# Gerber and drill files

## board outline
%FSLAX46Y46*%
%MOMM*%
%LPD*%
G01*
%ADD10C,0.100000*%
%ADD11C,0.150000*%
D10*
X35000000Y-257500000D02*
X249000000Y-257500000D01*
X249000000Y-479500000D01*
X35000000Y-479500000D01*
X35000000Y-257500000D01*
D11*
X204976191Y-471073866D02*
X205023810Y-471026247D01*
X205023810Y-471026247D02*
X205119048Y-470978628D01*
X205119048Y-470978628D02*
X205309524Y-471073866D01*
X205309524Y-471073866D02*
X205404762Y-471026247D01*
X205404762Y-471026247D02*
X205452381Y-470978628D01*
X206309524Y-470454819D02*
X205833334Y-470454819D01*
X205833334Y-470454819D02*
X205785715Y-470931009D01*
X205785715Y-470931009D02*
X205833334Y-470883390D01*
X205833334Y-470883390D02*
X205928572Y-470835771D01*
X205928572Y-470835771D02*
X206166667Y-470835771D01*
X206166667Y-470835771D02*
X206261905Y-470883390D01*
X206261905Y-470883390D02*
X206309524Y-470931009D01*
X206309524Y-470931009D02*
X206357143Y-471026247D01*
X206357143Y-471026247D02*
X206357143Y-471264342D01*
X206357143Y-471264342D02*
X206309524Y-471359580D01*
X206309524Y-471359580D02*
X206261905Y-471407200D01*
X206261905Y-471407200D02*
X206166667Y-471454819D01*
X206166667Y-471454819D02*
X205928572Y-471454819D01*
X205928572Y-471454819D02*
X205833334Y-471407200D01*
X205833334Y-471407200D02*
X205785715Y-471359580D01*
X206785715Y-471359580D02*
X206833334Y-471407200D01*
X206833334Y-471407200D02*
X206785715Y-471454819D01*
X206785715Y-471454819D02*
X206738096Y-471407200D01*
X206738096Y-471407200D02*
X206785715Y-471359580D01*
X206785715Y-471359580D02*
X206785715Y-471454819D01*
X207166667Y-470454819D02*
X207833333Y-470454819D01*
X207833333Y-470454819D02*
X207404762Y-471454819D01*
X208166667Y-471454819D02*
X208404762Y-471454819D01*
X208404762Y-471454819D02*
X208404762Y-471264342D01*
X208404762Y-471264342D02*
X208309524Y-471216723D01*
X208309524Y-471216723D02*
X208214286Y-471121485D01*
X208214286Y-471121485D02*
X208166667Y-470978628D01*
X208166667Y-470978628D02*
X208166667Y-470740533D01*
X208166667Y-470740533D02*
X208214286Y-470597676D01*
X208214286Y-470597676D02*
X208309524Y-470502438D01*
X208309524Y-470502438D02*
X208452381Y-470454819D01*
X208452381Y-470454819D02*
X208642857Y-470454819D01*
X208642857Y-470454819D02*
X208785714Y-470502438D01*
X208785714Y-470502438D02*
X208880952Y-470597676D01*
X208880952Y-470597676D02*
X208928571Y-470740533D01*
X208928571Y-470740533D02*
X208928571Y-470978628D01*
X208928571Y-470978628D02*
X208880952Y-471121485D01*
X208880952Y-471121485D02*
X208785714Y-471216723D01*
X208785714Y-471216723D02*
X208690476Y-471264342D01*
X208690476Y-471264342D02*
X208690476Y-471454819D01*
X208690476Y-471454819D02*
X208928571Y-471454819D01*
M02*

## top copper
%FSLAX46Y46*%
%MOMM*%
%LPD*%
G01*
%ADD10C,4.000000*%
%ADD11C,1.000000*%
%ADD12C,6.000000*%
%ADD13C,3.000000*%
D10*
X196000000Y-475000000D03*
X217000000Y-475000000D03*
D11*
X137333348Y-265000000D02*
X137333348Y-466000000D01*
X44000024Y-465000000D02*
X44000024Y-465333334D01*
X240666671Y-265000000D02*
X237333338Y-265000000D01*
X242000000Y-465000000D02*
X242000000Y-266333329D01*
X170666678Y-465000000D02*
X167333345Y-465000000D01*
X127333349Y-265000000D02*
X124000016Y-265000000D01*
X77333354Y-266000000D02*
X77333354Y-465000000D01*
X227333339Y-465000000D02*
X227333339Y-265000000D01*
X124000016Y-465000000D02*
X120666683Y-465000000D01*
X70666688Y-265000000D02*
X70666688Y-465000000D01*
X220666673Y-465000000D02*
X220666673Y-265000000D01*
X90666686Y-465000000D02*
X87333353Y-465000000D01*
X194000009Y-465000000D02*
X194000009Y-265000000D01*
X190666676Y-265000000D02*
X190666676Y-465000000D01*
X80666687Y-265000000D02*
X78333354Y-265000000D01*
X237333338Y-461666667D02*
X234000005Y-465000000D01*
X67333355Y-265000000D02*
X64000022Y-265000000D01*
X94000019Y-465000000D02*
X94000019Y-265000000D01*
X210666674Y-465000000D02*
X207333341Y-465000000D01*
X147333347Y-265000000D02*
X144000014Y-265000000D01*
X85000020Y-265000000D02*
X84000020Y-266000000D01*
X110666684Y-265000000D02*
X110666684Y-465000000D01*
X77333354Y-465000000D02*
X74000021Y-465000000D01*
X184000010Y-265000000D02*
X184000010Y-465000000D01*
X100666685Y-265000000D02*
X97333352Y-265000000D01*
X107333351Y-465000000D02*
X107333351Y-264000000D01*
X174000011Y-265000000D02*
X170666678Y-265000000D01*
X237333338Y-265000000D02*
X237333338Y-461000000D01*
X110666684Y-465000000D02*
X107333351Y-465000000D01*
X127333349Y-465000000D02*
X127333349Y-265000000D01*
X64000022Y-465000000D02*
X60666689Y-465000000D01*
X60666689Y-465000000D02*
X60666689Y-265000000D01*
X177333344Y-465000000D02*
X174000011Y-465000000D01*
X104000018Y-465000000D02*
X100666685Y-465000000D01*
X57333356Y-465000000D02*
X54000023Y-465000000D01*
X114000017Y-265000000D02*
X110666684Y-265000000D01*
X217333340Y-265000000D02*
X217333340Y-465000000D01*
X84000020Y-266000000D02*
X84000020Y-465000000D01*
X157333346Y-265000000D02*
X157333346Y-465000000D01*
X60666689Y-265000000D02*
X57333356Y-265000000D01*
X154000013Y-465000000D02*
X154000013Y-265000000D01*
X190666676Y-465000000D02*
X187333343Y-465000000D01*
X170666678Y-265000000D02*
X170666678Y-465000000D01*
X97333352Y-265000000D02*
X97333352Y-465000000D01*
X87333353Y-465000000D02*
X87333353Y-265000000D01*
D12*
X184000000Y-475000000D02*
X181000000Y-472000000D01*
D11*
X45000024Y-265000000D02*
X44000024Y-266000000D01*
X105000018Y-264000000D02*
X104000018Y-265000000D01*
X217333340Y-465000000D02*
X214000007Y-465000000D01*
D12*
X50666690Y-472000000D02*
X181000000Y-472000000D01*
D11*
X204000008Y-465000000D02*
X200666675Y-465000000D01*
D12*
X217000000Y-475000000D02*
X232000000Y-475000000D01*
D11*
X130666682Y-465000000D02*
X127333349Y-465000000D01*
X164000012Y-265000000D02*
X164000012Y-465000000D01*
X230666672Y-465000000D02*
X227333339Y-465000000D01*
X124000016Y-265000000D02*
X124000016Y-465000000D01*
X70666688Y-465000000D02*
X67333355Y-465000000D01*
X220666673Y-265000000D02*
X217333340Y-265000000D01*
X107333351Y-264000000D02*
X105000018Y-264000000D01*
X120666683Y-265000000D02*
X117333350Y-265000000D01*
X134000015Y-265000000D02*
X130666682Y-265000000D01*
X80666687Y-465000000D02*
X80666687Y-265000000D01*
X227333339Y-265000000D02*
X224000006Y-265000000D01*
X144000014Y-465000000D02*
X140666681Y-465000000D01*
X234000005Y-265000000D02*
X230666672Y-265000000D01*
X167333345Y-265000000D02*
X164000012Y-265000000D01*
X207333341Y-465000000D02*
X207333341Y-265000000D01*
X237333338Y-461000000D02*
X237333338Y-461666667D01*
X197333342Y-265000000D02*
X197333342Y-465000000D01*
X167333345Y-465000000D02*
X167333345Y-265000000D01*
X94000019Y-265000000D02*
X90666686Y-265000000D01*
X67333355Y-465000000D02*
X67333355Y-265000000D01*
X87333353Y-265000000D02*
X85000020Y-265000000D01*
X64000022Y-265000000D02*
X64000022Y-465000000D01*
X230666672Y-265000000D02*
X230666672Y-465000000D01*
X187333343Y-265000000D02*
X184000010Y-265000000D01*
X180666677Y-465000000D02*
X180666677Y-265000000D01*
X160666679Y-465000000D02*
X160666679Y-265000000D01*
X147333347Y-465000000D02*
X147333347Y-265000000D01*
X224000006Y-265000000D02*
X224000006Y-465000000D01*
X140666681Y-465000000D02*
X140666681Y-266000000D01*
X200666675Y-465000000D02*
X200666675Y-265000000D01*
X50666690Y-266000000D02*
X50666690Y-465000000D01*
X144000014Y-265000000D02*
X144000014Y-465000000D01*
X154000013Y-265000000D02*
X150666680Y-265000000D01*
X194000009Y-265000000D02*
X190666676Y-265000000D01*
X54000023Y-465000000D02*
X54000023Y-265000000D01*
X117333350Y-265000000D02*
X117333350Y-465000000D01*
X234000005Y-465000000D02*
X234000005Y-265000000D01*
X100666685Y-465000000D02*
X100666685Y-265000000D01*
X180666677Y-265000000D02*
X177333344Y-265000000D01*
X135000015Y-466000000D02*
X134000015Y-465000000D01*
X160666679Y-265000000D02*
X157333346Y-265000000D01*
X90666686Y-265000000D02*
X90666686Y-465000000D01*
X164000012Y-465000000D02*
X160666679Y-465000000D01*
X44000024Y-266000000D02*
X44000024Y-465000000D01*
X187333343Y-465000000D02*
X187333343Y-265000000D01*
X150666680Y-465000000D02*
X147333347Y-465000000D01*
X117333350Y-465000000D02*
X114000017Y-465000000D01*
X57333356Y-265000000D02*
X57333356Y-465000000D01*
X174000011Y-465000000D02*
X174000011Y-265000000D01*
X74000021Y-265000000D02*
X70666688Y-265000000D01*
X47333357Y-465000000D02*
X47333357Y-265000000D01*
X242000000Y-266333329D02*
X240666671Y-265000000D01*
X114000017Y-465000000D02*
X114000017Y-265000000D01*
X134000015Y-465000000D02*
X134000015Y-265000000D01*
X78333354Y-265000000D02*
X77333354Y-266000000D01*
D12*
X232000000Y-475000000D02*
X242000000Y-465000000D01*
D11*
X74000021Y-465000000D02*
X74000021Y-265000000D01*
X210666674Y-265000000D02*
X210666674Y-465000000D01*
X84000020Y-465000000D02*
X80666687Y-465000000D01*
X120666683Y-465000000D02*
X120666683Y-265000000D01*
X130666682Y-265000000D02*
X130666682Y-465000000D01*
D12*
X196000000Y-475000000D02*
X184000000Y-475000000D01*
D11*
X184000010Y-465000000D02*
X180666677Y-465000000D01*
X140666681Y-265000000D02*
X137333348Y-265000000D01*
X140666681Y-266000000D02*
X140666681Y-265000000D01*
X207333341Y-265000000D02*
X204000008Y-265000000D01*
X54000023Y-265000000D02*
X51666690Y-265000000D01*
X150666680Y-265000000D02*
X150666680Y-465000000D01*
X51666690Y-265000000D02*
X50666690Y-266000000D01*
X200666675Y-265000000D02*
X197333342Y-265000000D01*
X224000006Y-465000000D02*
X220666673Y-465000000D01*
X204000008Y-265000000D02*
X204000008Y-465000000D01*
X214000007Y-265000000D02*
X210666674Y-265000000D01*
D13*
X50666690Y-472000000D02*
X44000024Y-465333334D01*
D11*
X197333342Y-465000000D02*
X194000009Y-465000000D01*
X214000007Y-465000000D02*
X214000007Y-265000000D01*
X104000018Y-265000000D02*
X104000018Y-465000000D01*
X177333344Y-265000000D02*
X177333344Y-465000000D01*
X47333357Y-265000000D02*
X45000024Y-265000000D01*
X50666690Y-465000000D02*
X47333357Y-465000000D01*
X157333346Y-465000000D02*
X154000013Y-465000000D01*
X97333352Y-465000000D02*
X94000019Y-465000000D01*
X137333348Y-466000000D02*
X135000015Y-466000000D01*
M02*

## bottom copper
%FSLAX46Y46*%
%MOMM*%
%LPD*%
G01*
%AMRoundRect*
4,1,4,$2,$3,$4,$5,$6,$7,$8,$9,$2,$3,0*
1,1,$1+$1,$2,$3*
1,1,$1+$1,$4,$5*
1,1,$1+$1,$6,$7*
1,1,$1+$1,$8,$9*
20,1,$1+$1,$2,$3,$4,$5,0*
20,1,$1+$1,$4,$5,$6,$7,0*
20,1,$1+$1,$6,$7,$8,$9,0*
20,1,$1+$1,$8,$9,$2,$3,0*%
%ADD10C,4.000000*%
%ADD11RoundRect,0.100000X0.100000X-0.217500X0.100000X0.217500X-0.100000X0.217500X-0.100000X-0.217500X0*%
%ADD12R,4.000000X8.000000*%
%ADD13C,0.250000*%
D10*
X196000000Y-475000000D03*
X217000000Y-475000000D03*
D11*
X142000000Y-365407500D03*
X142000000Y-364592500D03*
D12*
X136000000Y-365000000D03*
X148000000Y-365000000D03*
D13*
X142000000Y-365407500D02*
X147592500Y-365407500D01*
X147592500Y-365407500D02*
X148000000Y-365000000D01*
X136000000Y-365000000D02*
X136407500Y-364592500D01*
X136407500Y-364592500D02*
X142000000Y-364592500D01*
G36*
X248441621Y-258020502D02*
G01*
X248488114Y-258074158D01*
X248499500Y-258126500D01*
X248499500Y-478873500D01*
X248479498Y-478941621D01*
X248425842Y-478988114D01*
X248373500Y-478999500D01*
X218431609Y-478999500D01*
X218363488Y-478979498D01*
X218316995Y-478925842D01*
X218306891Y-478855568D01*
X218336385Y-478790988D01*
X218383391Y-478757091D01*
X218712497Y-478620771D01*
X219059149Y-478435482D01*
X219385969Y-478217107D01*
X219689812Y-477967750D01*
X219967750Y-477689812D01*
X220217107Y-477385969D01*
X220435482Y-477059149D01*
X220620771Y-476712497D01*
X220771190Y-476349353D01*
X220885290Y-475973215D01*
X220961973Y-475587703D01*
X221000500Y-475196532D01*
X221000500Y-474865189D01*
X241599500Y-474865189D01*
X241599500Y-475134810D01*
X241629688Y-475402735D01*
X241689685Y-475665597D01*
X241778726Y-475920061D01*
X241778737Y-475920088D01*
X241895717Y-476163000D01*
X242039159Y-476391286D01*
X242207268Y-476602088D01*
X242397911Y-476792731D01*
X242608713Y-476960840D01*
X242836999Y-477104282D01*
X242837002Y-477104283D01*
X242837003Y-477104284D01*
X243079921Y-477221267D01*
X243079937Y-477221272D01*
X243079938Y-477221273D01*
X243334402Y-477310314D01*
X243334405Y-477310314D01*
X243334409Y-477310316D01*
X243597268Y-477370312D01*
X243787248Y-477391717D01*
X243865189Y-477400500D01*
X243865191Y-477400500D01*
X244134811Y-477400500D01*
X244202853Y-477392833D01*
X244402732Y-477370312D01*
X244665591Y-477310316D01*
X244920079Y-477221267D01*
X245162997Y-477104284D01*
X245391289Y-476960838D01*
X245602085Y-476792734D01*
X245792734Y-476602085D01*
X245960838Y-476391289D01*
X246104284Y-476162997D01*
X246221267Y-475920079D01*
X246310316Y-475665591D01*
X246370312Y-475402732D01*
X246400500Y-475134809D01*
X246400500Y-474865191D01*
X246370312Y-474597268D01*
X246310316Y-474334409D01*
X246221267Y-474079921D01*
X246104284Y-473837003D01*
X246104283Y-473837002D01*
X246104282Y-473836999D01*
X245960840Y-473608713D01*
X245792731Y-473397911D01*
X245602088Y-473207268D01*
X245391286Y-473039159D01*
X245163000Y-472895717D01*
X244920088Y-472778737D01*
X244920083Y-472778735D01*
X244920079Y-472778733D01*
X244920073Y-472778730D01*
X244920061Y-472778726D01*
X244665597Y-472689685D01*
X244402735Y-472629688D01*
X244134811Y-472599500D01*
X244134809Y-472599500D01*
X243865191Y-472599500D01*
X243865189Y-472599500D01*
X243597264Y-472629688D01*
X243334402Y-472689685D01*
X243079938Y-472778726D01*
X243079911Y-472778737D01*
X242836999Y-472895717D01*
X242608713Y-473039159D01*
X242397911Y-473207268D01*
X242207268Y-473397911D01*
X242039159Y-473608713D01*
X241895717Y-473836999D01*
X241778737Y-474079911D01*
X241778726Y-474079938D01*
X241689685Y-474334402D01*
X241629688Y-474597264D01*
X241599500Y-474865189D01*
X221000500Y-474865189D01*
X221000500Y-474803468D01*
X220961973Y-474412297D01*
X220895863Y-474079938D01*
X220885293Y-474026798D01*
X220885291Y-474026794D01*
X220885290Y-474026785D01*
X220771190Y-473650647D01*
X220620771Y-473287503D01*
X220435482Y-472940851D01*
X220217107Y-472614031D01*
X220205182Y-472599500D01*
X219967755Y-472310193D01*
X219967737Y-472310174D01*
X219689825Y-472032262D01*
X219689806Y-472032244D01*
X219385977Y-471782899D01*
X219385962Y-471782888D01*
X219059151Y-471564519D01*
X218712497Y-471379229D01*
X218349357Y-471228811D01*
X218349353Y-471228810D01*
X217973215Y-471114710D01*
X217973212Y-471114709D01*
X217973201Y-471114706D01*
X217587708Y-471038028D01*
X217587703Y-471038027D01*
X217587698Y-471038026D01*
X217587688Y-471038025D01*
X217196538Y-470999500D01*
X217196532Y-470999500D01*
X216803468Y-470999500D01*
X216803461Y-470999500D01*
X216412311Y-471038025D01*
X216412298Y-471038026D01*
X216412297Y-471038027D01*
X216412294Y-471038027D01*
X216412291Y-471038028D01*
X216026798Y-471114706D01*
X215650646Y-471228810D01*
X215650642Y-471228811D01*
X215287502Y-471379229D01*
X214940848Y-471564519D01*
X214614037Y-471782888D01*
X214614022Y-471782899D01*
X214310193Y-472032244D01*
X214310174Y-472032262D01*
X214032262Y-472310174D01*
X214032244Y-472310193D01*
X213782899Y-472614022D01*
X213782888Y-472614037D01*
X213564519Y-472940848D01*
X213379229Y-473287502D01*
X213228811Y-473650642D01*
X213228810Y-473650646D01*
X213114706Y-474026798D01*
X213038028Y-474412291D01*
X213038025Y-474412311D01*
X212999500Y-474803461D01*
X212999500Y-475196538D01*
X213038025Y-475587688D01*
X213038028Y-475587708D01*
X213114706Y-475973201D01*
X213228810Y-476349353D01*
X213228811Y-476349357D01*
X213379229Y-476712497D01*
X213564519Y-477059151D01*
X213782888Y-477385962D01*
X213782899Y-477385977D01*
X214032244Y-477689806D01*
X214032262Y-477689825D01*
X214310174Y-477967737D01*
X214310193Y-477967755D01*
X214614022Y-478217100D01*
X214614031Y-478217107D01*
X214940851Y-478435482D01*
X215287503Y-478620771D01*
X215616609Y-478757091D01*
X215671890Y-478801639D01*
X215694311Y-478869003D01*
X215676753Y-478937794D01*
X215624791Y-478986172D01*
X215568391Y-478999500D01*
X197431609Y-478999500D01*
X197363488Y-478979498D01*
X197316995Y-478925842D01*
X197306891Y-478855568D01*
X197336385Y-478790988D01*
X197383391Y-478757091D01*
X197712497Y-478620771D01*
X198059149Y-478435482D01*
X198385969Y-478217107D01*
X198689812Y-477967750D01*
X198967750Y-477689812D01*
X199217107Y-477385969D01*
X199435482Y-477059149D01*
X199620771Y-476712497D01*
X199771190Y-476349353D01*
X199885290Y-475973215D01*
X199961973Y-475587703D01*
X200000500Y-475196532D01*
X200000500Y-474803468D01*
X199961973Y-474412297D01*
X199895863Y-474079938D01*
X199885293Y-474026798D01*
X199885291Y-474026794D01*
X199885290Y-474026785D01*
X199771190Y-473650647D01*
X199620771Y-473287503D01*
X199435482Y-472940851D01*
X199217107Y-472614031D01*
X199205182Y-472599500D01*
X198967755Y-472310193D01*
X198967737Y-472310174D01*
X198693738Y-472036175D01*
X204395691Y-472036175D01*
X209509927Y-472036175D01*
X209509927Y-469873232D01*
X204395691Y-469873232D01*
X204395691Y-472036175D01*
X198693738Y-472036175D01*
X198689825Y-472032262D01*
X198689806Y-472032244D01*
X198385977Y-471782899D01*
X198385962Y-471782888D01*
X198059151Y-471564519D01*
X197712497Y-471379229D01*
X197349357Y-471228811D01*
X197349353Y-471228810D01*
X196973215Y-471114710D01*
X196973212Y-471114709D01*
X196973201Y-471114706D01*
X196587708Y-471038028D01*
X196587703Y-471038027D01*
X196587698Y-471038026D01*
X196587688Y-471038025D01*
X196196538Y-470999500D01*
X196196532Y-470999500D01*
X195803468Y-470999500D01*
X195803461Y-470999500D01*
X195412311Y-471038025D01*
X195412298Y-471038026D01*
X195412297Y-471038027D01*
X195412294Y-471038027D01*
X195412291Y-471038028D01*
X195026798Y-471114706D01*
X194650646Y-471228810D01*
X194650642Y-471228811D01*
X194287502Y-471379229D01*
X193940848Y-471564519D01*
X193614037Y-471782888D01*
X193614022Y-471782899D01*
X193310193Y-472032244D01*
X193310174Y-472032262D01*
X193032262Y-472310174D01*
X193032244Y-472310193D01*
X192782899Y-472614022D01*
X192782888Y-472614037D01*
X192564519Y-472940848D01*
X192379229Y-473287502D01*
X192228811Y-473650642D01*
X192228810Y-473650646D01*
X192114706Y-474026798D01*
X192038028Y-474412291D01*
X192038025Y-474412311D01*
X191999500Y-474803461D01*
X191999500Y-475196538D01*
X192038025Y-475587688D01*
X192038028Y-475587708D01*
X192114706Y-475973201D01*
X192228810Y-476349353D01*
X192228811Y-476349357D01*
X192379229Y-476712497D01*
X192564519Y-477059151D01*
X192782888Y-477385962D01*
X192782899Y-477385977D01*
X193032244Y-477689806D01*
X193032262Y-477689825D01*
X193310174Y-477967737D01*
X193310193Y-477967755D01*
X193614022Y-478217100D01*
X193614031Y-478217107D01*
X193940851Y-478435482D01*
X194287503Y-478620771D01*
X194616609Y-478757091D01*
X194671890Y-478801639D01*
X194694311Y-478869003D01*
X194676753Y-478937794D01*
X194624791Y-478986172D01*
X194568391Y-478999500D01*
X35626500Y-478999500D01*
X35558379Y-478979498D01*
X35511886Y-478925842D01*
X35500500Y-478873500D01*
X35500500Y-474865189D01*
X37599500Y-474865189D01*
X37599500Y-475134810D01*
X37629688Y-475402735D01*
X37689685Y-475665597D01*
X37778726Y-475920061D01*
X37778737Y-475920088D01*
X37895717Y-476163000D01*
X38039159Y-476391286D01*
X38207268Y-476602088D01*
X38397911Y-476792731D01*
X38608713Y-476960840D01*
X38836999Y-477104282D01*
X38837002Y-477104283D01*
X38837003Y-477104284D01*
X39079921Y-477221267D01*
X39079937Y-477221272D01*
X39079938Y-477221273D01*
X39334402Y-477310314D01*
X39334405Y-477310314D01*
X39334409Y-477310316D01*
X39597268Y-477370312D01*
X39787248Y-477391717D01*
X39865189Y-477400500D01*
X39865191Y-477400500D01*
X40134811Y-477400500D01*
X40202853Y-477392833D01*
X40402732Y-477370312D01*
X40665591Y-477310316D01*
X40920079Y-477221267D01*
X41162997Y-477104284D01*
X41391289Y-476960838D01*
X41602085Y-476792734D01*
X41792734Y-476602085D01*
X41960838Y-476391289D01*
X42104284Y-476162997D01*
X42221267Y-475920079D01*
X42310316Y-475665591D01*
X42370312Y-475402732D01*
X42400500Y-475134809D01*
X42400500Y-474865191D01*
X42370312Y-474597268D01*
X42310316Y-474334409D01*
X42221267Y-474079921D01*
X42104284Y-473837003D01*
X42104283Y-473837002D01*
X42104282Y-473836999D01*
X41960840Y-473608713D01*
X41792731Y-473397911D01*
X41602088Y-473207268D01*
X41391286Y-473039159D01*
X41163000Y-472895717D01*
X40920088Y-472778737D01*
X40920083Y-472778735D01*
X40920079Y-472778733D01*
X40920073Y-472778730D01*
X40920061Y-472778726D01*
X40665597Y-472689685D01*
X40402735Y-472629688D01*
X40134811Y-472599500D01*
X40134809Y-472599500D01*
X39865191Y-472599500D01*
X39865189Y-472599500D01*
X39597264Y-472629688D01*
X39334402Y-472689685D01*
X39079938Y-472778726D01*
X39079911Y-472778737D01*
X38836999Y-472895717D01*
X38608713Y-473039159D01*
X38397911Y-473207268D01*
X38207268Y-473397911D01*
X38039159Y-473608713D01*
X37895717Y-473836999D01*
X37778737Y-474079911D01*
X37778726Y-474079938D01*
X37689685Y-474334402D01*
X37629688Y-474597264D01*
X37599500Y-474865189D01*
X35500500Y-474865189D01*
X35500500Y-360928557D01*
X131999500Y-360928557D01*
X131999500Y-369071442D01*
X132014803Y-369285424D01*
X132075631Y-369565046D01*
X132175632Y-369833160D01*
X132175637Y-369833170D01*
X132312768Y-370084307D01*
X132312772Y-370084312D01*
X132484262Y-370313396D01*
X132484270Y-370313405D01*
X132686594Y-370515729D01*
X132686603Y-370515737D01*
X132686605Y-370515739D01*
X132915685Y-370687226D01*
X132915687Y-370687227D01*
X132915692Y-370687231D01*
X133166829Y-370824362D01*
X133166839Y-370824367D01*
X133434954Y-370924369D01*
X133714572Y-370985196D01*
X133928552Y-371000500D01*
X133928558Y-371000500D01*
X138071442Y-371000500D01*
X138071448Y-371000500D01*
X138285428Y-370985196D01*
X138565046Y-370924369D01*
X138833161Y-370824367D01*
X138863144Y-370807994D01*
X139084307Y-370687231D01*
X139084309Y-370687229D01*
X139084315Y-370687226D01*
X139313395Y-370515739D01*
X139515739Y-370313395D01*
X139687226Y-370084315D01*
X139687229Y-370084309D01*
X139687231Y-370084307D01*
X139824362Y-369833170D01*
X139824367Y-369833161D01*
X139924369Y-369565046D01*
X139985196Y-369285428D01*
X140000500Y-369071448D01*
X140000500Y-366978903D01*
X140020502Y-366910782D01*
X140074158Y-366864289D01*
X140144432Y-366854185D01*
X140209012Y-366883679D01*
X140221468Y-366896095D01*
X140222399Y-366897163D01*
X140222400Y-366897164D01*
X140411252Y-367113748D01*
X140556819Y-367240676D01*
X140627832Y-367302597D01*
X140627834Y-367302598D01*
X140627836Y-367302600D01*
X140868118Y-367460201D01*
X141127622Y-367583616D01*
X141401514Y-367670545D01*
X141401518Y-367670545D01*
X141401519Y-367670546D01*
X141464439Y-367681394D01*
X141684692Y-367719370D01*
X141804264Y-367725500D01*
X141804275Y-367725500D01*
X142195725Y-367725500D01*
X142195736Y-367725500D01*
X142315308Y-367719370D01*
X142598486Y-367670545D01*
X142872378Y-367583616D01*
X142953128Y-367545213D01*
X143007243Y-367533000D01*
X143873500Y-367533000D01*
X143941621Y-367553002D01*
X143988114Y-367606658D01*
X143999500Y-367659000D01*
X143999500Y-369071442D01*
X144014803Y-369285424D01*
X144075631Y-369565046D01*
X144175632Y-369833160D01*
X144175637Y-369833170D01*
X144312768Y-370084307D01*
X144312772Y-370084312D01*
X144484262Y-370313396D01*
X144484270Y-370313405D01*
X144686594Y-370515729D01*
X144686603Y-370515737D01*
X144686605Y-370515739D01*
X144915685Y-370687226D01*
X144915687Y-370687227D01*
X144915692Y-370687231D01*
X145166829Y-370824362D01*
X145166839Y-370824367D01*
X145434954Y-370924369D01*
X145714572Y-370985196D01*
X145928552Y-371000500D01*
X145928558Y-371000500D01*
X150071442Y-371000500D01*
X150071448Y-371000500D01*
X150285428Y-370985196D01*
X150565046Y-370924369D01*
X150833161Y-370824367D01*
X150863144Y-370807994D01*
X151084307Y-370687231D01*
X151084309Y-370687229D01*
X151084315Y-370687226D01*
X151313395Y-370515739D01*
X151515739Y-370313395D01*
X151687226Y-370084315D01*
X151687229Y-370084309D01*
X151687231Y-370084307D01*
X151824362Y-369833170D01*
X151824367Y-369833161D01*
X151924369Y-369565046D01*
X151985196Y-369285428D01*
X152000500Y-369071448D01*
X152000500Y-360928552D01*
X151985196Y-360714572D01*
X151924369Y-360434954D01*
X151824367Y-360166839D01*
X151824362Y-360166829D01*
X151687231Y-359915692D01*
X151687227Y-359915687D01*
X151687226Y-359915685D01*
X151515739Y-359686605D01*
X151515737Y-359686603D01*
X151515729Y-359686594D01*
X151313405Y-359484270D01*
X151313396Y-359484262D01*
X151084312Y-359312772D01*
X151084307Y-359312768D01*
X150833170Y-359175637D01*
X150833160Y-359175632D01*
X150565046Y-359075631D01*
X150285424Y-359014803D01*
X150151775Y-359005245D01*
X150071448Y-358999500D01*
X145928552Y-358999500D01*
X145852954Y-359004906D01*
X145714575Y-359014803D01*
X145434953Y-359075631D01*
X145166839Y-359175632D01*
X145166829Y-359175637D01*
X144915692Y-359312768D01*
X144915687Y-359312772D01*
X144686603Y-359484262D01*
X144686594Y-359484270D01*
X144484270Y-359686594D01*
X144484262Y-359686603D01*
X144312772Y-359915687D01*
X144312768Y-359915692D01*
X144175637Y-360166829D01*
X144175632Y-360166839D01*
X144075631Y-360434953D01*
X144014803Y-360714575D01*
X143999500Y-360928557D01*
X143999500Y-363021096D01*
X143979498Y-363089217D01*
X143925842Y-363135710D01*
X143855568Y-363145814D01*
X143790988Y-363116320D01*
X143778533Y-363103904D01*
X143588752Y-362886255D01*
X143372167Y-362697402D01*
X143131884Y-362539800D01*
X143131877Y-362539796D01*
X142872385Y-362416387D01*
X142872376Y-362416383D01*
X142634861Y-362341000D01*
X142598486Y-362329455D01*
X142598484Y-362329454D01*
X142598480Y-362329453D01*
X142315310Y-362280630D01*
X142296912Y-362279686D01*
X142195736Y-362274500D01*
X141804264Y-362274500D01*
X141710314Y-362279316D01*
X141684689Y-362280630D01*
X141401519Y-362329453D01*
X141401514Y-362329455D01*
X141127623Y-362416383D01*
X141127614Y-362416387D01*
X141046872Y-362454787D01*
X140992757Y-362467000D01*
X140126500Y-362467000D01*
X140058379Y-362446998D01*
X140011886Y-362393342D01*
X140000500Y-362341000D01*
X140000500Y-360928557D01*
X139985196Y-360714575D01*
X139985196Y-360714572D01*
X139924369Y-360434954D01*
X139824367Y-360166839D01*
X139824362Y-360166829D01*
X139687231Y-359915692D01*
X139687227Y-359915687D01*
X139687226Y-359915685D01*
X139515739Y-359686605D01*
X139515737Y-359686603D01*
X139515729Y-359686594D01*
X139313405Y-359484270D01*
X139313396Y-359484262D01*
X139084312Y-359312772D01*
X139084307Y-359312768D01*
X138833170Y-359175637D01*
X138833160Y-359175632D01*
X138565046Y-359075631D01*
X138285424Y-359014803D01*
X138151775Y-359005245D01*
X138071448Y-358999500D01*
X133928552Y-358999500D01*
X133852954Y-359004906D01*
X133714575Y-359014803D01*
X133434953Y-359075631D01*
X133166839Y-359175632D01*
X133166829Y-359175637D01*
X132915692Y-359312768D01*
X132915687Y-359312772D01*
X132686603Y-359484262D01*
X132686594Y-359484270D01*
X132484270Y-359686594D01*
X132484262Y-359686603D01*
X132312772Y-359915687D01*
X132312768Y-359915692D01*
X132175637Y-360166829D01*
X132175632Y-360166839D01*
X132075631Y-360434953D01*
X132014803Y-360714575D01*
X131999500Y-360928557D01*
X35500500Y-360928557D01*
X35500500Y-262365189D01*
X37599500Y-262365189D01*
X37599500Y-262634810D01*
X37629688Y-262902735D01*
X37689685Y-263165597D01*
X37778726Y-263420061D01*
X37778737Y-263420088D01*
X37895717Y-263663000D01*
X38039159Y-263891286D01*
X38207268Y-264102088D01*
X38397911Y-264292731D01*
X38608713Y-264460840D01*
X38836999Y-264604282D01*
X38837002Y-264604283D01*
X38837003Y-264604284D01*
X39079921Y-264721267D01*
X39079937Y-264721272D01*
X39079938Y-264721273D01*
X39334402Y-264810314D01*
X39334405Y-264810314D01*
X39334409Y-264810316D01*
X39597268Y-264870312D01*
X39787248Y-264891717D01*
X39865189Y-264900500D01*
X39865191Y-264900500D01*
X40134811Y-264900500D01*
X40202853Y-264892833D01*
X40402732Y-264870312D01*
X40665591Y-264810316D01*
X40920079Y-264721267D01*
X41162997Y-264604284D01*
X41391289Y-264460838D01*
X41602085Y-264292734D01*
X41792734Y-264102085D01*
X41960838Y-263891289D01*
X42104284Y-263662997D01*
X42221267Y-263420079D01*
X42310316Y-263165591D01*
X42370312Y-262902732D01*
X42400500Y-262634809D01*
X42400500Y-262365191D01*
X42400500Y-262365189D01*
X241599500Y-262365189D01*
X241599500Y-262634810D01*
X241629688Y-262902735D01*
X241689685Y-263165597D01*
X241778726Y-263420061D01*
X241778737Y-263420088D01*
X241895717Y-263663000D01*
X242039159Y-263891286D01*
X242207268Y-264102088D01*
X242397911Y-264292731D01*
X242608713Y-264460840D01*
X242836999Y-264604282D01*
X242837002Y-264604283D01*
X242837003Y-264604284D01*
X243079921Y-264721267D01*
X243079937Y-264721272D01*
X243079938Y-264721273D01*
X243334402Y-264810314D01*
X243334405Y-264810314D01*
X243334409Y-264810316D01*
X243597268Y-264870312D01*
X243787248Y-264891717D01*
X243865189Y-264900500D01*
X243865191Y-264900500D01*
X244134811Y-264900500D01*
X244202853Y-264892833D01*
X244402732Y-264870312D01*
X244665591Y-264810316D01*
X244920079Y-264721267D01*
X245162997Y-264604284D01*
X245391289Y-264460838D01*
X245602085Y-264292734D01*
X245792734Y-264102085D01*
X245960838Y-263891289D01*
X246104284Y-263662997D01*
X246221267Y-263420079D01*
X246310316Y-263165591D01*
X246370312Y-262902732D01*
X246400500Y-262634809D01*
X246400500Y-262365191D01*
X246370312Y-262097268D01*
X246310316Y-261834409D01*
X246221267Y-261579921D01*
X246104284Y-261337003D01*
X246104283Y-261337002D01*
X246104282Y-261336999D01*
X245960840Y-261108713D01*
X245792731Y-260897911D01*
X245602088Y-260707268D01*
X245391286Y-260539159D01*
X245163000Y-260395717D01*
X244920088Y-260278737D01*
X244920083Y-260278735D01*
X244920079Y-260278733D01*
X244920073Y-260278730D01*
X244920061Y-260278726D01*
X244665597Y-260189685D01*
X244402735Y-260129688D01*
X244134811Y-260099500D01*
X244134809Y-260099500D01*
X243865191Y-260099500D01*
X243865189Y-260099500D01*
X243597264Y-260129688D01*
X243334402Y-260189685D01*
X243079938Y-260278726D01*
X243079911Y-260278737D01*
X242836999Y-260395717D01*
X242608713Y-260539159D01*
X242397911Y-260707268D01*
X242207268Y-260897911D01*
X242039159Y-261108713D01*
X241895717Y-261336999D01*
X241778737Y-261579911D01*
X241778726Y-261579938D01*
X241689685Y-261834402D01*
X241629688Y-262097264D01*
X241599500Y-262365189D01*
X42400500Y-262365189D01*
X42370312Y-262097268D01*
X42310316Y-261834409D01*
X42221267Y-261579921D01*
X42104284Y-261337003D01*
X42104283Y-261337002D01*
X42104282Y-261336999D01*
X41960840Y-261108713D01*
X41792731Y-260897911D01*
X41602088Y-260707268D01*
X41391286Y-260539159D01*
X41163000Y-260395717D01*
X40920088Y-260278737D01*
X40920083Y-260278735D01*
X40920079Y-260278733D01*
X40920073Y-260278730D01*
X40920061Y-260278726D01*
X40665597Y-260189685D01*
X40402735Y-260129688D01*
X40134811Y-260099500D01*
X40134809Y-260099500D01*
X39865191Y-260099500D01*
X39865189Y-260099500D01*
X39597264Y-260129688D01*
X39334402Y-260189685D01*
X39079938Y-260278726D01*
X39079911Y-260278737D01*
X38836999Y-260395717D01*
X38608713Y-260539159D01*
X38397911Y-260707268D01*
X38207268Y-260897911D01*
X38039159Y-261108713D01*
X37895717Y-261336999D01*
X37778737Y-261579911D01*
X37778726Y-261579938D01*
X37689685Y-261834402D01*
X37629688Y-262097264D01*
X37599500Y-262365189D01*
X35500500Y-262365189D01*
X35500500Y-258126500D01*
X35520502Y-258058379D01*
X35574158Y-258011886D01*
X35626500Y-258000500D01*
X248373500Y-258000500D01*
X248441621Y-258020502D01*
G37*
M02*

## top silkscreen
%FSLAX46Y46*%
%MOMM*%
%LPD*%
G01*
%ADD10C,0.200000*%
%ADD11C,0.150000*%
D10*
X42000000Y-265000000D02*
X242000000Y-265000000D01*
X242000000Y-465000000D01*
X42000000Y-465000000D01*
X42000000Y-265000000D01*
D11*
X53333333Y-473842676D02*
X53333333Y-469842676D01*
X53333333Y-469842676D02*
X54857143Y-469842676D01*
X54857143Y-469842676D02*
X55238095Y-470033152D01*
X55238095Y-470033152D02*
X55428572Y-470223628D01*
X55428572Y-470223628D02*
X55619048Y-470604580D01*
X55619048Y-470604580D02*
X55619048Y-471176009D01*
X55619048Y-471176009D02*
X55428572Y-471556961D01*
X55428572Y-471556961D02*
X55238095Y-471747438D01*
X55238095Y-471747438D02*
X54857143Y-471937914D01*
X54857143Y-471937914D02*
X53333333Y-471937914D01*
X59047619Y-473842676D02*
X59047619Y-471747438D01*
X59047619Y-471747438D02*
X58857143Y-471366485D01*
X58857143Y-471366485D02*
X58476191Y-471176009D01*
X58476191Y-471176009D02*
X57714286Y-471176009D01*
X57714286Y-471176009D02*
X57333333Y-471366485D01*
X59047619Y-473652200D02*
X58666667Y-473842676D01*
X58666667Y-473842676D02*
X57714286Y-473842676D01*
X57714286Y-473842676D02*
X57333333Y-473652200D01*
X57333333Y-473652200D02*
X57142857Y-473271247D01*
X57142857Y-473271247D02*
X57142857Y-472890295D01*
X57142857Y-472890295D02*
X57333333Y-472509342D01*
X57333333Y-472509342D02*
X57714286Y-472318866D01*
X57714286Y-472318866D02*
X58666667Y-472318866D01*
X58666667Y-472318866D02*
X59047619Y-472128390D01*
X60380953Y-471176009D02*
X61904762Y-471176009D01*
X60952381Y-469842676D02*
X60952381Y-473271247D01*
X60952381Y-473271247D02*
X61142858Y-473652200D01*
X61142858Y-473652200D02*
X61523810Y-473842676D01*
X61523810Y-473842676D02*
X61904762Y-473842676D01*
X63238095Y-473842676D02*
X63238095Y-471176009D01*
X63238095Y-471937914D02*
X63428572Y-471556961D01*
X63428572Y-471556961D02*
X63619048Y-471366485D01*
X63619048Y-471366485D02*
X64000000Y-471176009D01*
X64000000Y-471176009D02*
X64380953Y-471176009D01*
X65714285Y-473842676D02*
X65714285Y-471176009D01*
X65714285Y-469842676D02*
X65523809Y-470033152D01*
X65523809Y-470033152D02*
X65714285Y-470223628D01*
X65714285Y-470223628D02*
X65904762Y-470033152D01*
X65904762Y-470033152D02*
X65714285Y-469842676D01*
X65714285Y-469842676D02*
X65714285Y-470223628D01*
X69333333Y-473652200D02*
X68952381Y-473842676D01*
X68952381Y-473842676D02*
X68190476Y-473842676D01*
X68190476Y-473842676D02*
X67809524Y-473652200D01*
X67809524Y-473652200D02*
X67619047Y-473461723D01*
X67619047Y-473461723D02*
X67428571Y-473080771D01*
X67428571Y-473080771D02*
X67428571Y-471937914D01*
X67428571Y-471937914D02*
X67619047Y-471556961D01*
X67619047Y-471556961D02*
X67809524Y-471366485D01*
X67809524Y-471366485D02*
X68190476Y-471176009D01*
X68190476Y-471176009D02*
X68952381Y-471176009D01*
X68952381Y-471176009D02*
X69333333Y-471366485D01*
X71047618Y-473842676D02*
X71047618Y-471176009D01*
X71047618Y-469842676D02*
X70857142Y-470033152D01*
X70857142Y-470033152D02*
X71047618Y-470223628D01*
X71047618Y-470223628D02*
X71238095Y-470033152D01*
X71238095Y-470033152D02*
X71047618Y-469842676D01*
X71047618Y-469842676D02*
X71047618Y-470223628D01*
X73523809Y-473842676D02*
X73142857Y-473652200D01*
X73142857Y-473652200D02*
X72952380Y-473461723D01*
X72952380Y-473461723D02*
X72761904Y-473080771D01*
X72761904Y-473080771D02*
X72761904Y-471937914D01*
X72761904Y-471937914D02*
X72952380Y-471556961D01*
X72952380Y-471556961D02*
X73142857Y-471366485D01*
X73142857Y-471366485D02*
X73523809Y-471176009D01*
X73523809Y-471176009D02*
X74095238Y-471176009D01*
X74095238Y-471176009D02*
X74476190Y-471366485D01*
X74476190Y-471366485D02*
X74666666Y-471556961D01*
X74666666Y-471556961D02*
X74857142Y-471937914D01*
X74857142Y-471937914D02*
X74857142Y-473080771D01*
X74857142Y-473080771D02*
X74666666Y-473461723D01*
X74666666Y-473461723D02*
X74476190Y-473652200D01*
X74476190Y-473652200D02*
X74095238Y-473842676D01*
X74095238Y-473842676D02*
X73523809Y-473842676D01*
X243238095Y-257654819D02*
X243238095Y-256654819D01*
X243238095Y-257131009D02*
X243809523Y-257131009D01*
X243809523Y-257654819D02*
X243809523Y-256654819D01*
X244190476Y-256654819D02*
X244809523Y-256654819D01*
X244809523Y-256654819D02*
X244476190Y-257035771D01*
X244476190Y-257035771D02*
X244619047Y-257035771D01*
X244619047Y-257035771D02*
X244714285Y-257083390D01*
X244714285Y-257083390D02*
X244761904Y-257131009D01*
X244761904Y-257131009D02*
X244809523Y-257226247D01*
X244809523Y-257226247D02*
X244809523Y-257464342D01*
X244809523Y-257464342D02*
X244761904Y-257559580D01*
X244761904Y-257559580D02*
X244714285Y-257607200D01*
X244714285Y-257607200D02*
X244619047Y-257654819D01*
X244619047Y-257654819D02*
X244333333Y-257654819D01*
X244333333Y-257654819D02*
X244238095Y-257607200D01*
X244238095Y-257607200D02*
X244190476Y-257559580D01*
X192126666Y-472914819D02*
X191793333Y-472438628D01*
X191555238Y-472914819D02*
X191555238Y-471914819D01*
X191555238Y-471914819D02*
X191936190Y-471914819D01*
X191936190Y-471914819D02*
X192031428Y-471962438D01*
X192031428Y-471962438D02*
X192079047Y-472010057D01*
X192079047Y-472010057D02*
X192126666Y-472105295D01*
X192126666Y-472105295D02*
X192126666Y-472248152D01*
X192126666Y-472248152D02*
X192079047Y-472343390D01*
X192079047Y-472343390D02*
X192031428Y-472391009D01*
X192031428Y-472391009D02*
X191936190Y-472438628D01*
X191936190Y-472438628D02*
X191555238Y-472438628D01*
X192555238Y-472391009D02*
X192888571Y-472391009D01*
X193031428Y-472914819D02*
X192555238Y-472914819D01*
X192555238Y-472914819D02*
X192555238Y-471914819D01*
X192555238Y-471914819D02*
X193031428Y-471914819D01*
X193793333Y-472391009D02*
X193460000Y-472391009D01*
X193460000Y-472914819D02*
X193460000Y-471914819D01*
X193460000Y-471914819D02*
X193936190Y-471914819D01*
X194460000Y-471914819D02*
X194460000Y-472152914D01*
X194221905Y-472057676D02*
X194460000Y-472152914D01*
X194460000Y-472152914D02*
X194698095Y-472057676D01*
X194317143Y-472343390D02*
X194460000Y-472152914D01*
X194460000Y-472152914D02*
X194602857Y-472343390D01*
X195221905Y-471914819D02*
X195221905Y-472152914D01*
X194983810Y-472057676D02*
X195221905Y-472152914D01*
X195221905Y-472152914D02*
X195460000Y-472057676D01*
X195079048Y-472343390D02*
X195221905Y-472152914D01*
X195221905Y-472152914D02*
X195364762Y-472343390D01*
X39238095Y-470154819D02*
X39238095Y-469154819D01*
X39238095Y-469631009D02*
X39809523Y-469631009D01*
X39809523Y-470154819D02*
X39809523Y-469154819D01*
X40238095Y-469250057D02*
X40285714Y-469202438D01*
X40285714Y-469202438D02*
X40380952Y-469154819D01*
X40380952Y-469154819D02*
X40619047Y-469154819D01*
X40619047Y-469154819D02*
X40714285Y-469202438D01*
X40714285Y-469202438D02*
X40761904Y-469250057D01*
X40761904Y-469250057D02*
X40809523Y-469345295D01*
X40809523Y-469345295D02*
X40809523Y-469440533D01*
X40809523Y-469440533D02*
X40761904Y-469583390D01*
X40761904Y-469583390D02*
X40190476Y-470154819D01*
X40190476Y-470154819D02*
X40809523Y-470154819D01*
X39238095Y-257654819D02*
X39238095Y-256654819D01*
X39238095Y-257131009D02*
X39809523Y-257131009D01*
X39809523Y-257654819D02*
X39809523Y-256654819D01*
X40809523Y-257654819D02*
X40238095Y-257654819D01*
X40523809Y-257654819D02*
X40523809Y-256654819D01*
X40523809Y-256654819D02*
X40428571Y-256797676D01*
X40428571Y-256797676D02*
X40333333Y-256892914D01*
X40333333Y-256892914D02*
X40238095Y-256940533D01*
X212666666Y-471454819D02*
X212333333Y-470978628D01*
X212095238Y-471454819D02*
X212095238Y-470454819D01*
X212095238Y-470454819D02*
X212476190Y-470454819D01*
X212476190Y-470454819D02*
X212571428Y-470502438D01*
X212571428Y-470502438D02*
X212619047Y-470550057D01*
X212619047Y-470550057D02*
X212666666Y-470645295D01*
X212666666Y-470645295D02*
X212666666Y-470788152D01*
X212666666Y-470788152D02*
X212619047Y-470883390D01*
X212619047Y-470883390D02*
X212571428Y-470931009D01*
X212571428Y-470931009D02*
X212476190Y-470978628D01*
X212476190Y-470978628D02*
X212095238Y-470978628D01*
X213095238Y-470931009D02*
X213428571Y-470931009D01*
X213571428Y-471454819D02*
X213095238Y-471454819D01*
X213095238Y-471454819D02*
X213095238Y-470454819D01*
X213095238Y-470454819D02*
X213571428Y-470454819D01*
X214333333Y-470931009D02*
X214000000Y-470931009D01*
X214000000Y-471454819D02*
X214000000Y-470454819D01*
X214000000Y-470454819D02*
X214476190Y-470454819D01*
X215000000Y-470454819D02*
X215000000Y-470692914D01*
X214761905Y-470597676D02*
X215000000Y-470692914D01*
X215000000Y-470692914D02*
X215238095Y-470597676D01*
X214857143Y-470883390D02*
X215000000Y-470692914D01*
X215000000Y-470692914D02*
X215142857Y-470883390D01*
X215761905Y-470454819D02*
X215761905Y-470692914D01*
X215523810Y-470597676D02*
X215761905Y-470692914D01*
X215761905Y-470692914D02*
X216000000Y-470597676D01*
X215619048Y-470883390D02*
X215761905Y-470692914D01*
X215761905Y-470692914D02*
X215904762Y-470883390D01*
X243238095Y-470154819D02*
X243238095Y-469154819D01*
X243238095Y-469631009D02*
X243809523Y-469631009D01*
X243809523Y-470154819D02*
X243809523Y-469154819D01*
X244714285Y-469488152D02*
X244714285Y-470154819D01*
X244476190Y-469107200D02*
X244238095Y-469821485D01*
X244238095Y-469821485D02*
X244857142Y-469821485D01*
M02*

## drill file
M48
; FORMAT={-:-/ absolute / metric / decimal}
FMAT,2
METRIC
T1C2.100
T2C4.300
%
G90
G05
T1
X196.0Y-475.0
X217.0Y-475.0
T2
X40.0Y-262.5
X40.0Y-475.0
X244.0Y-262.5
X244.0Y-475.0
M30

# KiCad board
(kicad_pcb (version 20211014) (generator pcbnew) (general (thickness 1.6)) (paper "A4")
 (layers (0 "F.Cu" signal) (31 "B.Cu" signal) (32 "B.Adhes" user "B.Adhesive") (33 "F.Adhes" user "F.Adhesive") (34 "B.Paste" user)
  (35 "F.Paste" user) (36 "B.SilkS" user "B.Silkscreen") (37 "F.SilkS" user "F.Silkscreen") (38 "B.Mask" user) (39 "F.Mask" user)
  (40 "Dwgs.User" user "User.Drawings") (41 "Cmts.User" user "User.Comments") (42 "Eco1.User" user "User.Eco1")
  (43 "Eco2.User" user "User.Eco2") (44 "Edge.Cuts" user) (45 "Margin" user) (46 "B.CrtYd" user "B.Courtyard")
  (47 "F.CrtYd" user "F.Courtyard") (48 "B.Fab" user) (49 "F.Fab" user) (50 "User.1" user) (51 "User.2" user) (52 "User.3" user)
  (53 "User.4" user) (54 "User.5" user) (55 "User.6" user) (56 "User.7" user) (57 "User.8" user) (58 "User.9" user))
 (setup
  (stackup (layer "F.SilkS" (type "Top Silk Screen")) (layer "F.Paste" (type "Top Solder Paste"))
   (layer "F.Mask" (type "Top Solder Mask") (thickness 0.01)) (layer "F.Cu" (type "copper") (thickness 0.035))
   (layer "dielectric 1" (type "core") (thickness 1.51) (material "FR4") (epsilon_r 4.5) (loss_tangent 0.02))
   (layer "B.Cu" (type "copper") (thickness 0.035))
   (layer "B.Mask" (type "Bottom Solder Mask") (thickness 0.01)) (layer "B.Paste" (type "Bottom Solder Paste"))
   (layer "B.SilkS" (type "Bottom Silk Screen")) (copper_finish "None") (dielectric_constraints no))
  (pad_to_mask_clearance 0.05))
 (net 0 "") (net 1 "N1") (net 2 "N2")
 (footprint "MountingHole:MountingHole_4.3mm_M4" (layer "F.Cu") (at 244 262.5)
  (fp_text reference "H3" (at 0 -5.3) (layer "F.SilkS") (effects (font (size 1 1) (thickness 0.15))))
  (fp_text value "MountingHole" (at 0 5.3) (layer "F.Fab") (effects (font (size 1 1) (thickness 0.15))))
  (pad "" np_thru_hole circle (at 0 0) (size 4.3 4.3) (drill 4.3) (layers *.Cu *.Mask)))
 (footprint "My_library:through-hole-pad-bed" (layer "F.Cu") (at 196 475)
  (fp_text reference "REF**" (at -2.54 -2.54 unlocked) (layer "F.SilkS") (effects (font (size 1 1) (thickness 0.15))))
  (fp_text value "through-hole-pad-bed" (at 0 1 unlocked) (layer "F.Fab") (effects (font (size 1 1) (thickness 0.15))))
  (pad "1" thru_hole circle (at 0 0) (size 4 4) (drill 2.1) (layers *.Cu *.Mask)))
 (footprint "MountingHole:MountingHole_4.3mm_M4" (layer "F.Cu") (at 40 475)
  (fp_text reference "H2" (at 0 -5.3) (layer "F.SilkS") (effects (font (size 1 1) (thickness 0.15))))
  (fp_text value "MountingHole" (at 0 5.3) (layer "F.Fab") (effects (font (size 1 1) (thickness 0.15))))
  (pad "" np_thru_hole circle (at 0 0) (size 4.3 4.3) (drill 4.3) (layers *.Cu *.Mask)))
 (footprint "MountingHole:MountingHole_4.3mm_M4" (layer "F.Cu") (at 40 262.5)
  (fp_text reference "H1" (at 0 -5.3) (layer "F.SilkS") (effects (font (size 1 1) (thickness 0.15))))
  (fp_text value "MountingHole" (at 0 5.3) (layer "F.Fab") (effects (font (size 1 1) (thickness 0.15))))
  (pad "" np_thru_hole circle (at 0 0) (size 4.3 4.3) (drill 4.3) (layers *.Cu *.Mask)))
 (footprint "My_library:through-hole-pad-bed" (layer "F.Cu") (at 217 475)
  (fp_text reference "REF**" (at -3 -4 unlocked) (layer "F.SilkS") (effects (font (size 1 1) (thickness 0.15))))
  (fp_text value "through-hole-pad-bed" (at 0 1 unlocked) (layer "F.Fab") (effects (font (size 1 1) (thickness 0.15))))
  (pad "1" thru_hole circle (at 0 0) (size 4 4) (drill 2.1) (layers *.Cu *.Mask)))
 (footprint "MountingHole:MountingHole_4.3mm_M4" (layer "F.Cu") (at 244 475)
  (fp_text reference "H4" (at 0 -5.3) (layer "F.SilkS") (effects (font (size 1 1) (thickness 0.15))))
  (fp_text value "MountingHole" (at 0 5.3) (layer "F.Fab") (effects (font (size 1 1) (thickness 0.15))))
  (pad "" np_thru_hole circle (at 0 0) (size 4.3 4.3) (drill 4.3) (layers *.Cu *.Mask)))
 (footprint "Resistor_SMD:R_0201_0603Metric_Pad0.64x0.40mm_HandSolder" (layer "B.Cu") (at 142 365 90)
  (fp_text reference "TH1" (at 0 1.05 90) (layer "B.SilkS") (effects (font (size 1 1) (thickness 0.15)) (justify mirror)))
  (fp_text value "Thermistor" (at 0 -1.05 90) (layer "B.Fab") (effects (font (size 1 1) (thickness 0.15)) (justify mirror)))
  (pad "" smd roundrect (at 0.4325 0 90) (size 0.458 0.36) (layers "B.Paste") (roundrect_rratio 0.25))
  (pad "" smd roundrect (at -0.4325 0 90) (size 0.458 0.36) (layers "B.Paste") (roundrect_rratio 0.25))
  (pad "1" smd roundrect (at -0.4075 0 90) (size 0.635 0.4) (layers "B.Cu" "B.Mask") (roundrect_rratio 0.25) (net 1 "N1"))
  (pad "2" smd roundrect (at 0.4075 0 90) (size 0.635 0.4) (layers "B.Cu" "B.Mask") (roundrect_rratio 0.25) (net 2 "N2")))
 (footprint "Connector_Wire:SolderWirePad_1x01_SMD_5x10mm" (layer "B.Cu") (at 136 365 180)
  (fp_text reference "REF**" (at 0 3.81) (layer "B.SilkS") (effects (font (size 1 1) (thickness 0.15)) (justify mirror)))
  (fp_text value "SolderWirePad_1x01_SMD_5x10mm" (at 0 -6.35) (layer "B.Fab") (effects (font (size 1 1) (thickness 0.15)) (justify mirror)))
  (pad "1" smd rect (at 0 0 180) (size 4 8) (layers "B.Cu" "B.Paste" "B.Mask") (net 2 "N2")))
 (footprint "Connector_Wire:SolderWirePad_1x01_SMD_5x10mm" (layer "B.Cu") (at 148 365 180)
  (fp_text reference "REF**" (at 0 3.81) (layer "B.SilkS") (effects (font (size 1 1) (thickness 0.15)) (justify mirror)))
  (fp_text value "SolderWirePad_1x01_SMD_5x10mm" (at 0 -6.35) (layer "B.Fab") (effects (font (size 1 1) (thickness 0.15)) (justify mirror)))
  (pad "1" smd rect (at 0 0 180) (size 4 8) (layers "B.Cu" "B.Paste" "B.Mask") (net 1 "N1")))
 (gr_rect (start 42 465) (end 242 265) (layer "F.SilkS") (width 0.2) (fill none))
 (gr_rect (start 249 257.5) (end 35 479.5) (layer "Edge.Cuts") (width 0.1) (fill none))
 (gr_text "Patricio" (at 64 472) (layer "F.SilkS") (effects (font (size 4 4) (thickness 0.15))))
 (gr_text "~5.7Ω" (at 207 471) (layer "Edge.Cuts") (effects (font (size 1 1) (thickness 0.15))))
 (segment (start 137.333348 265) (end 137.333348 466) (width 1) (layer "F.Cu") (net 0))
 (segment (start 44.000024 465) (end 44.000024 465.333334) (width 1) (layer "F.Cu") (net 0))
 (segment (start 240.666671 265) (end 237.333338 265) (width 1) (layer "F.Cu") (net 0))
 (segment (start 242 465) (end 242 266.333329) (width 1) (layer "F.Cu") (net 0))
 (segment (start 170.666678 465) (end 167.333345 465) (width 1) (layer "F.Cu") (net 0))
 (segment (start 127.333349 265) (end 124.000016 265) (width 1) (layer "F.Cu") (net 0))
 (segment (start 77.333354 266) (end 77.333354 465) (width 1) (layer "F.Cu") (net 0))
 (segment (start 227.333339 465) (end 227.333339 265) (width 1) (layer "F.Cu") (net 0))
 (segment (start 124.000016 465) (end 120.666683 465) (width 1) (layer "F.Cu") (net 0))
 (segment (start 70.666688 265) (end 70.666688 465) (width 1) (layer "F.Cu") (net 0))
 (segment (start 220.666673 465) (end 220.666673 265) (width 1) (layer "F.Cu") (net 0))
 (segment (start 90.666686 465) (end 87.333353 465) (width 1) (layer "F.Cu") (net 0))
 (segment (start 194.000009 465) (end 194.000009 265) (width 1) (layer "F.Cu") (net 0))
 (segment (start 190.666676 265) (end 190.666676 465) (width 1) (layer "F.Cu") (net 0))
 (segment (start 80.666687 265) (end 78.333354 265) (width 1) (layer "F.Cu") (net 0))
 (segment (start 237.333338 461.666667) (end 234.000005 465) (width 1) (layer "F.Cu") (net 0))
 (segment (start 67.333355 265) (end 64.000022 265) (width 1) (layer "F.Cu") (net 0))
 (segment (start 94.000019 465) (end 94.000019 265) (width 1) (layer "F.Cu") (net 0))
 (segment (start 210.666674 465) (end 207.333341 465) (width 1) (layer "F.Cu") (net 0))
 (segment (start 147.333347 265) (end 144.000014 265) (width 1) (layer "F.Cu") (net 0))
 (segment (start 85.00002 265) (end 84.00002 266) (width 1) (layer "F.Cu") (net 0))
 (segment (start 110.666684 265) (end 110.666684 465) (width 1) (layer "F.Cu") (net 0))
 (segment (start 77.333354 465) (end 74.000021 465) (width 1) (layer "F.Cu") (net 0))
 (segment (start 184.00001 265) (end 184.00001 465) (width 1) (layer "F.Cu") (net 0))
 (segment (start 100.666685 265) (end 97.333352 265) (width 1) (layer "F.Cu") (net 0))
 (segment (start 107.333351 465) (end 107.333351 264) (width 1) (layer "F.Cu") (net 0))
 (segment (start 174.000011 265) (end 170.666678 265) (width 1) (layer "F.Cu") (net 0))
 (segment (start 237.333338 265) (end 237.333338 461) (width 1) (layer "F.Cu") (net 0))
 (segment (start 110.666684 465) (end 107.333351 465) (width 1) (layer "F.Cu") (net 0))
 (segment (start 127.333349 465) (end 127.333349 265) (width 1) (layer "F.Cu") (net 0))
 (segment (start 64.000022 465) (end 60.666689 465) (width 1) (layer "F.Cu") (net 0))
 (segment (start 60.666689 465) (end 60.666689 265) (width 1) (layer "F.Cu") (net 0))
 (segment (start 177.333344 465) (end 174.000011 465) (width 1) (layer "F.Cu") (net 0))
 (segment (start 104.000018 465) (end 100.666685 465) (width 1) (layer "F.Cu") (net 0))
 (segment (start 57.333356 465) (end 54.000023 465) (width 1) (layer "F.Cu") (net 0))
 (segment (start 114.000017 265) (end 110.666684 265) (width 1) (layer "F.Cu") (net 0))
 (segment (start 217.33334 265) (end 217.33334 465) (width 1) (layer "F.Cu") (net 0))
 (segment (start 84.00002 266) (end 84.00002 465) (width 1) (layer "F.Cu") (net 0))
 (segment (start 157.333346 265) (end 157.333346 465) (width 1) (layer "F.Cu") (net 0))
 (segment (start 60.666689 265) (end 57.333356 265) (width 1) (layer "F.Cu") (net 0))
 (segment (start 154.000013 465) (end 154.000013 265) (width 1) (layer "F.Cu") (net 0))
 (segment (start 190.666676 465) (end 187.333343 465) (width 1) (layer "F.Cu") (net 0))
 (segment (start 170.666678 265) (end 170.666678 465) (width 1) (layer "F.Cu") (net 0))
 (segment (start 97.333352 265) (end 97.333352 465) (width 1) (layer "F.Cu") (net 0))
 (segment (start 87.333353 465) (end 87.333353 265) (width 1) (layer "F.Cu") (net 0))
 (segment (start 184 475) (end 181 472) (width 6) (layer "F.Cu") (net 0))
 (segment (start 45.000024 265) (end 44.000024 266) (width 1) (layer "F.Cu") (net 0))
 (segment (start 105.000018 264) (end 104.000018 265) (width 1) (layer "F.Cu") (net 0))
 (segment (start 217.33334 465) (end 214.000007 465) (width 1) (layer "F.Cu") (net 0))
 (segment (start 50.66669 472) (end 181 472) (width 6) (layer "F.Cu") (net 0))
 (segment (start 204.000008 465) (end 200.666675 465) (width 1) (layer "F.Cu") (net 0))
 (segment (start 217 475) (end 232 475) (width 6) (layer "F.Cu") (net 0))
 (segment (start 130.666682 465) (end 127.333349 465) (width 1) (layer "F.Cu") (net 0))
 (segment (start 164.000012 265) (end 164.000012 465) (width 1) (layer "F.Cu") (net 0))
 (segment (start 230.666672 465) (end 227.333339 465) (width 1) (layer "F.Cu") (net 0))
 (segment (start 124.000016 265) (end 124.000016 465) (width 1) (layer "F.Cu") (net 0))
 (segment (start 70.666688 465) (end 67.333355 465) (width 1) (layer "F.Cu") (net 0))
 (segment (start 220.666673 265) (end 217.33334 265) (width 1) (layer "F.Cu") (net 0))
 (segment (start 107.333351 264) (end 105.000018 264) (width 1) (layer "F.Cu") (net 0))
 (segment (start 120.666683 265) (end 117.33335 265) (width 1) (layer "F.Cu") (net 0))
 (segment (start 134.000015 265) (end 130.666682 265) (width 1) (layer "F.Cu") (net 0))
 (segment (start 80.666687 465) (end 80.666687 265) (width 1) (layer "F.Cu") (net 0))
 (segment (start 227.333339 265) (end 224.000006 265) (width 1) (layer "F.Cu") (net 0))
 (segment (start 144.000014 465) (end 140.666681 465) (width 1) (layer "F.Cu") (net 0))
 (segment (start 234.000005 265) (end 230.666672 265) (width 1) (layer "F.Cu") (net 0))
 (segment (start 167.333345 265) (end 164.000012 265) (width 1) (layer "F.Cu") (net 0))
 (segment (start 207.333341 465) (end 207.333341 265) (width 1) (layer "F.Cu") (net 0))
 (segment (start 237.333338 461) (end 237.333338 461.666667) (width 1) (layer "F.Cu") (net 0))
 (segment (start 197.333342 265) (end 197.333342 465) (width 1) (layer "F.Cu") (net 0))
 (segment (start 167.333345 465) (end 167.333345 265) (width 1) (layer "F.Cu") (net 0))
 (segment (start 94.000019 265) (end 90.666686 265) (width 1) (layer "F.Cu") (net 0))
 (segment (start 67.333355 465) (end 67.333355 265) (width 1) (layer "F.Cu") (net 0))
 (segment (start 87.333353 265) (end 85.00002 265) (width 1) (layer "F.Cu") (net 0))
 (segment (start 64.000022 265) (end 64.000022 465) (width 1) (layer "F.Cu") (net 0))
 (segment (start 230.666672 265) (end 230.666672 465) (width 1) (layer "F.Cu") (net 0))
 (segment (start 187.333343 265) (end 184.00001 265) (width 1) (layer "F.Cu") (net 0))
 (segment (start 180.666677 465) (end 180.666677 265) (width 1) (layer "F.Cu") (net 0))
 (segment (start 160.666679 465) (end 160.666679 265) (width 1) (layer "F.Cu") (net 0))
 (segment (start 147.333347 465) (end 147.333347 265) (width 1) (layer "F.Cu") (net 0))
 (segment (start 224.000006 265) (end 224.000006 465) (width 1) (layer "F.Cu") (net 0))
 (segment (start 140.666681 465) (end 140.666681 266) (width 1) (layer "F.Cu") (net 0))
 (segment (start 200.666675 465) (end 200.666675 265) (width 1) (layer "F.Cu") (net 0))
 (segment (start 50.66669 266) (end 50.66669 465) (width 1) (layer "F.Cu") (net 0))
 (segment (start 144.000014 265) (end 144.000014 465) (width 1) (layer "F.Cu") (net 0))
 (segment (start 154.000013 265) (end 150.66668 265) (width 1) (layer "F.Cu") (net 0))
 (segment (start 194.000009 265) (end 190.666676 265) (width 1) (layer "F.Cu") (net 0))
 (segment (start 54.000023 465) (end 54.000023 265) (width 1) (layer "F.Cu") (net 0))
 (segment (start 117.33335 265) (end 117.33335 465) (width 1) (layer "F.Cu") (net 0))
 (segment (start 234.000005 465) (end 234.000005 265) (width 1) (layer "F.Cu") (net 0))
 (segment (start 100.666685 465) (end 100.666685 265) (width 1) (layer "F.Cu") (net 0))
 (segment (start 180.666677 265) (end 177.333344 265) (width 1) (layer "F.Cu") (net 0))
 (segment (start 135.000015 466) (end 134.000015 465) (width 1) (layer "F.Cu") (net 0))
 (segment (start 160.666679 265) (end 157.333346 265) (width 1) (layer "F.Cu") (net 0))
 (segment (start 90.666686 265) (end 90.666686 465) (width 1) (layer "F.Cu") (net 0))
 (segment (start 164.000012 465) (end 160.666679 465) (width 1) (layer "F.Cu") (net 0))
 (segment (start 44.000024 266) (end 44.000024 465) (width 1) (layer "F.Cu") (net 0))
 (segment (start 187.333343 465) (end 187.333343 265) (width 1) (layer "F.Cu") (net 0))
 (segment (start 150.66668 465) (end 147.333347 465) (width 1) (layer "F.Cu") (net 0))
 (segment (start 117.33335 465) (end 114.000017 465) (width 1) (layer "F.Cu") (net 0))
 (segment (start 57.333356 265) (end 57.333356 465) (width 1) (layer "F.Cu") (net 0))
 (segment (start 174.000011 465) (end 174.000011 265) (width 1) (layer "F.Cu") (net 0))
 (segment (start 74.000021 265) (end 70.666688 265) (width 1) (layer "F.Cu") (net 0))
 (segment (start 47.333357 465) (end 47.333357 265) (width 1) (layer "F.Cu") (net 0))
 (segment (start 242 266.333329) (end 240.666671 265) (width 1) (layer "F.Cu") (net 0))
 (segment (start 114.000017 465) (end 114.000017 265) (width 1) (layer "F.Cu") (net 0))
 (segment (start 134.000015 465) (end 134.000015 265) (width 1) (layer "F.Cu") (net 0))
 (segment (start 78.333354 265) (end 77.333354 266) (width 1) (layer "F.Cu") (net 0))
 (segment (start 232 475) (end 242 465) (width 6) (layer "F.Cu") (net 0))
 (segment (start 74.000021 465) (end 74.000021 265) (width 1) (layer "F.Cu") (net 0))
 (segment (start 210.666674 265) (end 210.666674 465) (width 1) (layer "F.Cu") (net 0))
 (segment (start 84.00002 465) (end 80.666687 465) (width 1) (layer "F.Cu") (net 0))
 (segment (start 120.666683 465) (end 120.666683 265) (width 1) (layer "F.Cu") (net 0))
 (segment (start 130.666682 265) (end 130.666682 465) (width 1) (layer "F.Cu") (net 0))
 (segment (start 196 475) (end 184 475) (width 6) (layer "F.Cu") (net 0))
 (segment (start 184.00001 465) (end 180.666677 465) (width 1) (layer "F.Cu") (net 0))
 (segment (start 140.666681 265) (end 137.333348 265) (width 1) (layer "F.Cu") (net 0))
 (segment (start 140.666681 266) (end 140.666681 265) (width 1) (layer "F.Cu") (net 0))
 (segment (start 207.333341 265) (end 204.000008 265) (width 1) (layer "F.Cu") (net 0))
 (segment (start 54.000023 265) (end 51.66669 265) (width 1) (layer "F.Cu") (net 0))
 (segment (start 150.66668 265) (end 150.66668 465) (width 1) (layer "F.Cu") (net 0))
 (segment (start 51.66669 265) (end 50.66669 266) (width 1) (layer "F.Cu") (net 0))
 (segment (start 200.666675 265) (end 197.333342 265) (width 1) (layer "F.Cu") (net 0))
 (segment (start 224.000006 465) (end 220.666673 465) (width 1) (layer "F.Cu") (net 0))
 (segment (start 204.000008 265) (end 204.000008 465) (width 1) (layer "F.Cu") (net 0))
 (segment (start 214.000007 265) (end 210.666674 265) (width 1) (layer "F.Cu") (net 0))
 (segment (start 50.66669 472) (end 44.000024 465.333334) (width 3) (layer "F.Cu") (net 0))
 (segment (start 197.333342 465) (end 194.000009 465) (width 1) (layer "F.Cu") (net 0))
 (segment (start 214.000007 465) (end 214.000007 265) (width 1) (layer "F.Cu") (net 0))
 (segment (start 104.000018 265) (end 104.000018 465) (width 1) (layer "F.Cu") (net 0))
 (segment (start 177.333344 265) (end 177.333344 465) (width 1) (layer "F.Cu") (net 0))
 (segment (start 47.333357 265) (end 45.000024 265) (width 1) (layer "F.Cu") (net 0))
 (segment (start 50.66669 465) (end 47.333357 465) (width 1) (layer "F.Cu") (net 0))
 (segment (start 157.333346 465) (end 154.000013 465) (width 1) (layer "F.Cu") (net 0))
 (segment (start 97.333352 465) (end 94.000019 465) (width 1) (layer "F.Cu") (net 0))
 (segment (start 137.333348 466) (end 135.000015 466) (width 1) (layer "F.Cu") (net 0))
 (segment (start 142 365.4075) (end 147.5925 365.4075) (width 0.25) (layer "B.Cu") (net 1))
 (segment (start 147.5925 365.4075) (end 148 365) (width 0.25) (layer "B.Cu") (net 1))
 (segment (start 136 365) (end 136.4075 364.5925) (width 0.25) (layer "B.Cu") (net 2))
 (segment (start 136.4075 364.5925) (end 142 364.5925) (width 0.25) (layer "B.Cu") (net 2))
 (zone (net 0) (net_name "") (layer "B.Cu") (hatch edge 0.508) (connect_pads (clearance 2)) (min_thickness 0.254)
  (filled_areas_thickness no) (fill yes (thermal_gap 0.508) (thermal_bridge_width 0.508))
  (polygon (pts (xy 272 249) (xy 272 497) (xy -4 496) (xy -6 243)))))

